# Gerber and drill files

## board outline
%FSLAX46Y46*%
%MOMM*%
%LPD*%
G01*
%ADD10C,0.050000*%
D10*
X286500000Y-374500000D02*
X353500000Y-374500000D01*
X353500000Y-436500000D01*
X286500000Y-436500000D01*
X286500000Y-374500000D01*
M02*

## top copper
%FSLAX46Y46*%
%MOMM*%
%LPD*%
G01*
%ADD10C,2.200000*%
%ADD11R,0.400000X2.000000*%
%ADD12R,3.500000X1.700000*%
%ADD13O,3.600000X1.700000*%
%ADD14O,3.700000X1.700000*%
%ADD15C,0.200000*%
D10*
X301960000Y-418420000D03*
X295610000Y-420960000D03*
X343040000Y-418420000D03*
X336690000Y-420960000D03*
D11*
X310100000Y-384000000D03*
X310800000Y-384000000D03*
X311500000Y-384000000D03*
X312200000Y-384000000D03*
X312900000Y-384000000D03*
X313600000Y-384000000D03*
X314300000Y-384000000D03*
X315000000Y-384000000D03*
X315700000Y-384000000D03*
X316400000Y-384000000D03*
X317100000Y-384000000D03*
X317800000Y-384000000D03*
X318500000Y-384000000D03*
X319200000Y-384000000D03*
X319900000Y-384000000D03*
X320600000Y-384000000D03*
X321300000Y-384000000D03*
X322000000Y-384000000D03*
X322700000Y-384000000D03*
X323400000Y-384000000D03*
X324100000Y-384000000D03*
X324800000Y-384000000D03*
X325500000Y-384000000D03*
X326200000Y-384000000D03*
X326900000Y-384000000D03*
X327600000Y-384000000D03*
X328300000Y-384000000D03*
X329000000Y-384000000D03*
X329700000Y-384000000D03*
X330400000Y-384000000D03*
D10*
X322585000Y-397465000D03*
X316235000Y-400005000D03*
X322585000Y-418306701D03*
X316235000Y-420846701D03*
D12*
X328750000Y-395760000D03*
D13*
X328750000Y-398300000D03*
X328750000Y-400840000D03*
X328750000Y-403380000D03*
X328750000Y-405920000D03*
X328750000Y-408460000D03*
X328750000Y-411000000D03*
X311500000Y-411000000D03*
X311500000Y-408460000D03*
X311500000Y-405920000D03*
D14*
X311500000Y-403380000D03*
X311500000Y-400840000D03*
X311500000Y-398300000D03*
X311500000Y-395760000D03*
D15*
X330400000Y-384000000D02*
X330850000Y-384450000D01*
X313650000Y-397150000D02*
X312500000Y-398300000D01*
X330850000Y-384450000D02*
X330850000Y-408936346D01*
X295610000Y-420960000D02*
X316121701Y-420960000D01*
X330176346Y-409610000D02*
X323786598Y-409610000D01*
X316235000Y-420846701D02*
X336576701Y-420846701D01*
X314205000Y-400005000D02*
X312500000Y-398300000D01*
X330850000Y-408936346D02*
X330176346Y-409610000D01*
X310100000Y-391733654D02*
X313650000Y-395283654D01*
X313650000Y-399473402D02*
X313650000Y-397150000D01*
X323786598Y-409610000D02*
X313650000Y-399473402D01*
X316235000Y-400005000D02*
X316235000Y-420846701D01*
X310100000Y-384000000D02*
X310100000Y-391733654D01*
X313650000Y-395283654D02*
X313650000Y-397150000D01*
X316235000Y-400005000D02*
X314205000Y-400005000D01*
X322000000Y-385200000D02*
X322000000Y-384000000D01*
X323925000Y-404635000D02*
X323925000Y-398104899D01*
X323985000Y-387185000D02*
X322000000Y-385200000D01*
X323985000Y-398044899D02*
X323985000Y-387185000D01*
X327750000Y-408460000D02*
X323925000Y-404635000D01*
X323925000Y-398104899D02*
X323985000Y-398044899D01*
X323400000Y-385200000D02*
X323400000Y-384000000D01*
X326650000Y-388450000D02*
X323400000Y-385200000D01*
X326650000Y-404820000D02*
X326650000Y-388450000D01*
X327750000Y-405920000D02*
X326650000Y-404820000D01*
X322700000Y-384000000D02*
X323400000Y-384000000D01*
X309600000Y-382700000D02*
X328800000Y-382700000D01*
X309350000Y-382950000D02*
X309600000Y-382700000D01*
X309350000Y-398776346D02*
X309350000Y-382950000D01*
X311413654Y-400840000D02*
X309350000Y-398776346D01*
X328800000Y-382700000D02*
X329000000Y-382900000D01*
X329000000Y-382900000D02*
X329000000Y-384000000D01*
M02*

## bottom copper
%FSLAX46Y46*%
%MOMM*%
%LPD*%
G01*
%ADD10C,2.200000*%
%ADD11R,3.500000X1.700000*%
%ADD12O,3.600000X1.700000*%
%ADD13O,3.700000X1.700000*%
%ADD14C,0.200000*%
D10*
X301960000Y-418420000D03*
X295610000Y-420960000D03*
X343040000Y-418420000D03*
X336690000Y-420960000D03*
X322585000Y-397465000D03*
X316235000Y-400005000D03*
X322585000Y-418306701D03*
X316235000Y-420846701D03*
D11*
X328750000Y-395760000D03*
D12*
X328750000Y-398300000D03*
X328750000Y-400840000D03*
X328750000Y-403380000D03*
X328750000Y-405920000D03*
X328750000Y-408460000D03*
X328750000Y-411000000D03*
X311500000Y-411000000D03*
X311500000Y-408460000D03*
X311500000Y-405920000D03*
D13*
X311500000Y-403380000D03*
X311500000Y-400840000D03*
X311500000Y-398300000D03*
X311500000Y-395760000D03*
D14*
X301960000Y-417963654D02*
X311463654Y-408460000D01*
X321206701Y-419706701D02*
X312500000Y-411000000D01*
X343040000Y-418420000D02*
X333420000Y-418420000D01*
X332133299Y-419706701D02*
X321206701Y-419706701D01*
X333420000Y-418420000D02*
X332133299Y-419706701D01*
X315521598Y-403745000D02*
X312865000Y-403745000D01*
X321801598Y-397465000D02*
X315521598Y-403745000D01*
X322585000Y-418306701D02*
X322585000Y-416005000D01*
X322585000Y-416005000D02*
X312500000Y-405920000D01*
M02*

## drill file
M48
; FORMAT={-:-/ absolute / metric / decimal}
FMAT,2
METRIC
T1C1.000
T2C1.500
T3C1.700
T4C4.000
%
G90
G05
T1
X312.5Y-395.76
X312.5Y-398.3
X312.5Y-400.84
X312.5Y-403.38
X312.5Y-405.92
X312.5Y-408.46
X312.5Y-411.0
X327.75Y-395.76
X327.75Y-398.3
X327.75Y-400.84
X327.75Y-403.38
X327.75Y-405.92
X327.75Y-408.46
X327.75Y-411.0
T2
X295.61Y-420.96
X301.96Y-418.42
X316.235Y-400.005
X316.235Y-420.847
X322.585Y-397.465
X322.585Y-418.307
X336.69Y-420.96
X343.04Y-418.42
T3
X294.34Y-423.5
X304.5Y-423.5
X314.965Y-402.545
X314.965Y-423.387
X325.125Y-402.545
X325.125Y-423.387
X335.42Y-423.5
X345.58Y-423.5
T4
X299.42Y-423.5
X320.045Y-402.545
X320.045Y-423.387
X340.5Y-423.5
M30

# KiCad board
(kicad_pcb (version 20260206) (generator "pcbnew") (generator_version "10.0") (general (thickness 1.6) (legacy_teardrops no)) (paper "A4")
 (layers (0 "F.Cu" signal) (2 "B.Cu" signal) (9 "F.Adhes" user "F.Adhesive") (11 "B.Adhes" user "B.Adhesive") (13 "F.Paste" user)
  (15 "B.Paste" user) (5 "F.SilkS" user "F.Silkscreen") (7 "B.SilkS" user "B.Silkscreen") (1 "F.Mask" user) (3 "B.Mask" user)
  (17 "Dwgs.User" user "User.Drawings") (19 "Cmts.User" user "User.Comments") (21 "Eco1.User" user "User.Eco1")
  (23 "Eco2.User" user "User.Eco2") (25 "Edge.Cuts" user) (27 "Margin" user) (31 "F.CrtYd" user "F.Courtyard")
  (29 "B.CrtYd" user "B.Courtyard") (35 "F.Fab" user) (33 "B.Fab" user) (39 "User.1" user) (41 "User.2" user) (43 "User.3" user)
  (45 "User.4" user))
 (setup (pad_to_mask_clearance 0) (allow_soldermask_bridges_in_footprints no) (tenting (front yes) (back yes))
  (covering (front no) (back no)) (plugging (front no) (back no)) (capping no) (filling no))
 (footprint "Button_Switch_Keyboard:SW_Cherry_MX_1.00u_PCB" (layer "F.Cu") (at 301.96 418.42)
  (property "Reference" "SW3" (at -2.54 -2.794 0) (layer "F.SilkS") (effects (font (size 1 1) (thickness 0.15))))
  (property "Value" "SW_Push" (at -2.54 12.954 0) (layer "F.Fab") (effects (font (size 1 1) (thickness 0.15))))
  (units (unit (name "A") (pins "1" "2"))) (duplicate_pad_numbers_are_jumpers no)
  (pad "" np_thru_hole circle (at -7.62 5.08) (size 1.7 1.7) (drill 1.7) (layers "*.Cu" "*.Mask"))
  (pad "" np_thru_hole circle (at -2.54 5.08) (size 4 4) (drill 4) (layers "*.Cu" "*.Mask"))
  (pad "" np_thru_hole circle (at 2.54 5.08) (size 1.7 1.7) (drill 1.7) (layers "*.Cu" "*.Mask"))
  (pad "1" thru_hole circle (at 0 0) (size 2.2 2.2) (drill 1.5) (layers "*.Cu" "*.Mask") (remove_unused_layers no)
   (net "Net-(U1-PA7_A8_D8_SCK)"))
  (pad "2" thru_hole circle (at -6.35 2.54) (size 2.2 2.2) (drill 1.5) (layers "*.Cu" "*.Mask") (remove_unused_layers no) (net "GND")))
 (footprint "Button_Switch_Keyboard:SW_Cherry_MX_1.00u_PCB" (layer "F.Cu") (at 343.04 418.42)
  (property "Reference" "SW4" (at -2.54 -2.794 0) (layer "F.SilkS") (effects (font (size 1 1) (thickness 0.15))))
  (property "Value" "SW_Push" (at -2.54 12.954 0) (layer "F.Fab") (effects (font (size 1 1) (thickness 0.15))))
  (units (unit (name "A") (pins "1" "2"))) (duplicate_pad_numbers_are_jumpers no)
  (pad "" np_thru_hole circle (at -7.62 5.08) (size 1.7 1.7) (drill 1.7) (layers "*.Cu" "*.Mask"))
  (pad "" np_thru_hole circle (at -2.54 5.08) (size 4 4) (drill 4) (layers "*.Cu" "*.Mask"))
  (pad "" np_thru_hole circle (at 2.54 5.08) (size 1.7 1.7) (drill 1.7) (layers "*.Cu" "*.Mask"))
  (pad "1" thru_hole circle (at 0 0) (size 2.2 2.2) (drill 1.5) (layers "*.Cu" "*.Mask") (remove_unused_layers no)
   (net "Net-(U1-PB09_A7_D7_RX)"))
  (pad "2" thru_hole circle (at -6.35 2.54) (size 2.2 2.2) (drill 1.5) (layers "*.Cu" "*.Mask") (remove_unused_layers no) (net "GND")))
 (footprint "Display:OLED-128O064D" (layer "F.Cu") (at 320.25 384)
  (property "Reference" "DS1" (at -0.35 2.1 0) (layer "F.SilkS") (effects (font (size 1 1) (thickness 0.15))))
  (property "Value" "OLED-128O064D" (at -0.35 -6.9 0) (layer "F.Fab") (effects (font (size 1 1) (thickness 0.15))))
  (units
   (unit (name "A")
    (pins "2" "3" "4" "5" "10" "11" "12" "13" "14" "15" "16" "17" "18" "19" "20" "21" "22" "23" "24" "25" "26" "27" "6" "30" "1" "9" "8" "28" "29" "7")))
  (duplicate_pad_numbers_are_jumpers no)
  (pad "1" smd rect (at -10.15 0) (size 0.4 2) (layers "F.Cu" "F.Mask" "F.Paste") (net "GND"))
  (pad "2" smd rect (at -9.45 0) (size 0.4 2) (layers "F.Cu" "F.Mask" "F.Paste") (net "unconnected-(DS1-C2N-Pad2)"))
  (pad "3" smd rect (at -8.75 0) (size 0.4 2) (layers "F.Cu" "F.Mask" "F.Paste") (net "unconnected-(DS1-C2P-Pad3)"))
  (pad "4" smd rect (at -8.05 0) (size 0.4 2) (layers "F.Cu" "F.Mask" "F.Paste") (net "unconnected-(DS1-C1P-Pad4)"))
  (pad "5" smd rect (at -7.35 0) (size 0.4 2) (layers "F.Cu" "F.Mask" "F.Paste") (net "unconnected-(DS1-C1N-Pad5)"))
  (pad "6" smd rect (at -6.65 0) (size 0.4 2) (layers "F.Cu" "F.Mask" "F.Paste") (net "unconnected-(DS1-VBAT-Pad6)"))
  (pad "7" smd rect (at -5.95 0) (size 0.4 2) (layers "F.Cu" "F.Mask" "F.Paste") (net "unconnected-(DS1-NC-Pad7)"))
  (pad "8" smd rect (at -5.25 0) (size 0.4 2) (layers "F.Cu" "F.Mask" "F.Paste") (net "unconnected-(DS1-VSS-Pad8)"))
  (pad "9" smd rect (at -4.55 0) (size 0.4 2) (layers "F.Cu" "F.Mask" "F.Paste") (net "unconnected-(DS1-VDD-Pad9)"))
  (pad "10" smd rect (at -3.85 0) (size 0.4 2) (layers "F.Cu" "F.Mask" "F.Paste") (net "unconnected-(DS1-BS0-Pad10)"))
  (pad "11" smd rect (at -3.15 0) (size 0.4 2) (layers "F.Cu" "F.Mask" "F.Paste") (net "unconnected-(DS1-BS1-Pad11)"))
  (pad "12" smd rect (at -2.45 0) (size 0.4 2) (layers "F.Cu" "F.Mask" "F.Paste") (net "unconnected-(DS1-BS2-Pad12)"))
  (pad "13" smd rect (at -1.75 0) (size 0.4 2) (layers "F.Cu" "F.Mask" "F.Paste") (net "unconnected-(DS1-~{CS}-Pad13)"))
  (pad "14" smd rect (at -1.05 0) (size 0.4 2) (layers "F.Cu" "F.Mask" "F.Paste") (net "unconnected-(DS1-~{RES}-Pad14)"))
  (pad "15" smd rect (at -0.35 0) (size 0.4 2) (layers "F.Cu" "F.Mask" "F.Paste") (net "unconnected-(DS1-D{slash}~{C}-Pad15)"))
  (pad "16" smd rect (at 0.35 0) (size 0.4 2) (layers "F.Cu" "F.Mask" "F.Paste") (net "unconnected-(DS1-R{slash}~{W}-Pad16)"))
  (pad "17" smd rect (at 1.05 0) (size 0.4 2) (layers "F.Cu" "F.Mask" "F.Paste") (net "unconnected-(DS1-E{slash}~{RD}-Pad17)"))
  (pad "18" smd rect (at 1.75 0) (size 0.4 2) (layers "F.Cu" "F.Mask" "F.Paste") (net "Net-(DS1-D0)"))
  (pad "19" smd rect (at 2.45 0) (size 0.4 2) (layers "F.Cu" "F.Mask" "F.Paste") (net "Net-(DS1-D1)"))
  (pad "20" smd rect (at 3.15 0) (size 0.4 2) (layers "F.Cu" "F.Mask" "F.Paste") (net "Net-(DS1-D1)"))
  (pad "21" smd rect (at 3.85 0) (size 0.4 2) (layers "F.Cu" "F.Mask" "F.Paste") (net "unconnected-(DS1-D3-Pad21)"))
  (pad "22" smd rect (at 4.55 0) (size 0.4 2) (layers "F.Cu" "F.Mask" "F.Paste") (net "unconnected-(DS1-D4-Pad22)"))
  (pad "23" smd rect (at 5.25 0) (size 0.4 2) (layers "F.Cu" "F.Mask" "F.Paste") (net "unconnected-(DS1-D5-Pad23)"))
  (pad "24" smd rect (at 5.95 0) (size 0.4 2) (layers "F.Cu" "F.Mask" "F.Paste") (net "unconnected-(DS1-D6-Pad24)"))
  (pad "25" smd rect (at 6.65 0) (size 0.4 2) (layers "F.Cu" "F.Mask" "F.Paste") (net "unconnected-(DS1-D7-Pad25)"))
  (pad "26" smd rect (at 7.35 0) (size 0.4 2) (layers "F.Cu" "F.Mask" "F.Paste") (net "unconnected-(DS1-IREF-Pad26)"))
  (pad "27" smd rect (at 8.05 0) (size 0.4 2) (layers "F.Cu" "F.Mask" "F.Paste") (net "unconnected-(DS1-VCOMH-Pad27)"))
  (pad "28" smd rect (at 8.75 0) (size 0.4 2) (layers "F.Cu" "F.Mask" "F.Paste") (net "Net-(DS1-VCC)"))
  (pad "29" smd rect (at 9.45 0) (size 0.4 2) (layers "F.Cu" "F.Mask" "F.Paste") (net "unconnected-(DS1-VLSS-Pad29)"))
  (pad "30" smd rect (at 10.15 0) (size 0.4 2) (layers "F.Cu" "F.Mask" "F.Paste") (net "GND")))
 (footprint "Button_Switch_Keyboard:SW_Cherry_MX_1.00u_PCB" (layer "F.Cu") (at 322.585 397.465)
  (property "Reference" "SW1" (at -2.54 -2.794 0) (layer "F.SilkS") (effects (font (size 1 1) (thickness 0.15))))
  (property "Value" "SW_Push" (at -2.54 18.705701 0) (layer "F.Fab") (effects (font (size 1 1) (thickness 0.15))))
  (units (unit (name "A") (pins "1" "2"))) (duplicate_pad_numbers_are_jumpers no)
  (pad "" np_thru_hole circle (at -7.62 5.08) (size 1.7 1.7) (drill 1.7) (layers "*.Cu" "*.Mask"))
  (pad "" np_thru_hole circle (at -2.54 5.08) (size 4 4) (drill 4) (layers "*.Cu" "*.Mask"))
  (pad "" np_thru_hole circle (at 2.54 5.08) (size 1.7 1.7) (drill 1.7) (layers "*.Cu" "*.Mask"))
  (pad "1" thru_hole circle (at 0 0) (size 2.2 2.2) (drill 1.5) (layers "*.Cu" "*.Mask") (remove_unused_layers no)
   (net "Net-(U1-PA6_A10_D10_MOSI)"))
  (pad "2" thru_hole circle (at -6.35 2.54) (size 2.2 2.2) (drill 1.5) (layers "*.Cu" "*.Mask") (remove_unused_layers no) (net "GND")))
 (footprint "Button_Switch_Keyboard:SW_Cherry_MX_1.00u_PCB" (layer "F.Cu") (at 322.585 418.306701)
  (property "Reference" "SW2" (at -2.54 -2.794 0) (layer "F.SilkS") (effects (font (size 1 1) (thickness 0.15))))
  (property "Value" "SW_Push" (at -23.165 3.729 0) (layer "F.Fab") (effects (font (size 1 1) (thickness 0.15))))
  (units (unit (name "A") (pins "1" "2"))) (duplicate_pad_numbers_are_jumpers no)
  (pad "" np_thru_hole circle (at -7.62 5.08) (size 1.7 1.7) (drill 1.7) (layers "*.Cu" "*.Mask"))
  (pad "" np_thru_hole circle (at -2.54 5.08) (size 4 4) (drill 4) (layers "*.Cu" "*.Mask"))
  (pad "" np_thru_hole circle (at 2.54 5.08) (size 1.7 1.7) (drill 1.7) (layers "*.Cu" "*.Mask"))
  (pad "1" thru_hole circle (at 0 0) (size 2.2 2.2) (drill 1.5) (layers "*.Cu" "*.Mask") (remove_unused_layers no)
   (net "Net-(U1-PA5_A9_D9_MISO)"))
  (pad "2" thru_hole circle (at -6.35 2.54) (size 2.2 2.2) (drill 1.5) (layers "*.Cu" "*.Mask") (remove_unused_layers no) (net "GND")))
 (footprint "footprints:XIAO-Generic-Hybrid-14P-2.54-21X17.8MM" (layer "B.Cu") (at 320.125 403.38 180)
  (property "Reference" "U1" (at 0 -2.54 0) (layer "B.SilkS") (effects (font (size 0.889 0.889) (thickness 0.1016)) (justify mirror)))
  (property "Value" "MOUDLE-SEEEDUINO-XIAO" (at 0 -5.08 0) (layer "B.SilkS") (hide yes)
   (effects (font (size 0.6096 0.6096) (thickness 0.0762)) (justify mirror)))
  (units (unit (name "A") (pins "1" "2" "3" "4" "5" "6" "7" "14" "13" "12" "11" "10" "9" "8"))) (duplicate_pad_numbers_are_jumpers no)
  (pad "1" thru_hole rect (at -7.625 7.62 180) (size 3.5 1.7) (drill 1 (offset -1 0)) (layers "*.Cu" "*.Mask") (remove_unused_layers no)
   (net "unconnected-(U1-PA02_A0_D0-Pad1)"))
  (pad "2" thru_hole oval (at -7.625 5.08 180) (size 3.6 1.7) (drill 1 (offset -1 0)) (layers "*.Cu" "*.Mask") (remove_unused_layers no)
   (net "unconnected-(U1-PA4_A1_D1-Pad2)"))
  (pad "3" thru_hole oval (at -7.625 2.54 180) (size 3.6 1.7) (drill 1 (offset -1 0)) (layers "*.Cu" "*.Mask") (remove_unused_layers no)
   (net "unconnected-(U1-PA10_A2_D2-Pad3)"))
  (pad "4" thru_hole oval (at -7.625 0 180) (size 3.6 1.7) (drill 1 (offset -1 0)) (layers "*.Cu" "*.Mask") (remove_unused_layers no)
   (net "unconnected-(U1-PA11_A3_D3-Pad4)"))
  (pad "5" thru_hole oval (at -7.625 -2.54 180) (size 3.6 1.7) (drill 1 (offset -1 0)) (layers "*.Cu" "*.Mask") (remove_unused_layers no)
   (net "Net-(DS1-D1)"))
  (pad "6" thru_hole oval (at -7.625 -5.08) (size 3.6 1.7) (drill 1 (offset 1 0)) (layers "*.Cu" "*.Mask") (remove_unused_layers no)
   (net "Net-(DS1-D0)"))
  (pad "7" thru_hole oval (at -7.625 -7.62 180) (size 3.6 1.7) (drill 1 (offset -1 0)) (layers "*.Cu" "*.Mask") (remove_unused_layers no)
   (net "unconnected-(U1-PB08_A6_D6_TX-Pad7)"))
  (pad "8" thru_hole oval (at 7.625 -7.62 180) (size 3.6 1.7) (drill 1 (offset 1 0)) (layers "*.Cu" "*.Mask") (remove_unused_layers no)
   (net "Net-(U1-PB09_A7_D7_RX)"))
  (pad "9" thru_hole oval (at 7.625 -5.08 180) (size 3.6 1.7) (drill 1 (offset 1 0)) (layers "*.Cu" "*.Mask") (remove_unused_layers no)
   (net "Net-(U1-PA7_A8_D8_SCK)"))
  (pad "10" thru_hole oval (at 7.625 -2.54 180) (size 3.6 1.7) (drill 1 (offset 1 0)) (layers "*.Cu" "*.Mask") (remove_unused_layers no)
   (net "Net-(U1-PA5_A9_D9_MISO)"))
  (pad "11" thru_hole oval (at 7.625 0 180) (size 3.7 1.7) (drill 1 (offset 1 0)) (layers "*.Cu" "*.Mask") (remove_unused_layers no)
   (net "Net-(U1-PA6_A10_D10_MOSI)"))
  (pad "12" thru_hole oval (at 7.625 2.54 180) (size 3.7 1.7) (drill 1 (offset 1 0)) (layers "*.Cu" "*.Mask") (remove_unused_layers no)
   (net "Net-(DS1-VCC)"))
  (pad "13" thru_hole oval (at 7.625 5.08 180) (size 3.7 1.7) (drill 1 (offset 1 0)) (layers "*.Cu" "*.Mask") (remove_unused_layers no)
   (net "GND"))
  (pad "14" thru_hole oval (at 7.625 7.62 180) (size 3.7 1.7) (drill 1 (offset 1 0)) (layers "*.Cu" "*.Mask") (remove_unused_layers no)
   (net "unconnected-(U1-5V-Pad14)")))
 (gr_rect (start 286.5 374.5) (end 353.5 436.5) (stroke (width 0.05) (type default)) (fill no) (layer "Edge.Cuts"))
 (segment (start 301.96 417.963654) (end 311.463654 408.46) (width 0.2) (layer "B.Cu") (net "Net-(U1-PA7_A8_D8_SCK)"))
 (segment (start 330.4 384) (end 330.85 384.45) (width 0.2) (layer "F.Cu") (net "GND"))
 (segment (start 313.65 397.15) (end 312.5 398.3) (width 0.2) (layer "F.Cu") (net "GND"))
 (segment (start 330.85 384.45) (end 330.85 408.936346) (width 0.2) (layer "F.Cu") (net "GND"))
 (segment (start 295.61 420.96) (end 316.121701 420.96) (width 0.2) (layer "F.Cu") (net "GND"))
 (segment (start 330.176346 409.61) (end 323.786598 409.61) (width 0.2) (layer "F.Cu") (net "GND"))
 (segment (start 316.235 420.846701) (end 336.576701 420.846701) (width 0.2) (layer "F.Cu") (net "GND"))
 (segment (start 314.205 400.005) (end 312.5 398.3) (width 0.2) (layer "F.Cu") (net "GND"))
 (segment (start 330.85 408.936346) (end 330.176346 409.61) (width 0.2) (layer "F.Cu") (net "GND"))
 (segment (start 310.1 391.733654) (end 313.65 395.283654) (width 0.2) (layer "F.Cu") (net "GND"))
 (segment (start 313.65 399.473402) (end 313.65 397.15) (width 0.2) (layer "F.Cu") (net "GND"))
 (segment (start 323.786598 409.61) (end 313.65 399.473402) (width 0.2) (layer "F.Cu") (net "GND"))
 (segment (start 316.235 400.005) (end 316.235 420.846701) (width 0.2) (layer "F.Cu") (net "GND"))
 (segment (start 310.1 384) (end 310.1 391.733654) (width 0.2) (layer "F.Cu") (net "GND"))
 (segment (start 313.65 395.283654) (end 313.65 397.15) (width 0.2) (layer "F.Cu") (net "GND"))
 (segment (start 316.235 400.005) (end 314.205 400.005) (width 0.2) (layer "F.Cu") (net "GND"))
 (segment (start 321.206701 419.706701) (end 312.5 411) (width 0.2) (layer "B.Cu") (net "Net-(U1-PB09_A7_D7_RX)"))
 (segment (start 343.04 418.42) (end 333.42 418.42) (width 0.2) (layer "B.Cu") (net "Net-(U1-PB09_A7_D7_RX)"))
 (segment (start 332.133299 419.706701) (end 321.206701 419.706701) (width 0.2) (layer "B.Cu") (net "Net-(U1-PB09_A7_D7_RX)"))
 (segment (start 333.42 418.42) (end 332.133299 419.706701) (width 0.2) (layer "B.Cu") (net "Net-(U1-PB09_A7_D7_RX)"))
 (segment (start 322 385.2) (end 322 384) (width 0.2) (layer "F.Cu") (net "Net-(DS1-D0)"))
 (segment (start 323.925 404.635) (end 323.925 398.104899) (width 0.2) (layer "F.Cu") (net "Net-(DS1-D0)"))
 (segment (start 323.985 387.185) (end 322 385.2) (width 0.2) (layer "F.Cu") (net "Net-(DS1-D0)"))
 (segment (start 323.985 398.044899) (end 323.985 387.185) (width 0.2) (layer "F.Cu") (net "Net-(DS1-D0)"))
 (segment (start 327.75 408.46) (end 323.925 404.635) (width 0.2) (layer "F.Cu") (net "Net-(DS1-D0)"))
 (segment (start 323.925 398.104899) (end 323.985 398.044899) (width 0.2) (layer "F.Cu") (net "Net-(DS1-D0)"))
 (segment (start 323.4 385.2) (end 323.4 384) (width 0.2) (layer "F.Cu") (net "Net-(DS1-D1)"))
 (segment (start 326.65 388.45) (end 323.4 385.2) (width 0.2) (layer "F.Cu") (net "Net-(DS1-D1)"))
 (segment (start 326.65 404.82) (end 326.65 388.45) (width 0.2) (layer "F.Cu") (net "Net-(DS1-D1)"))
 (segment (start 327.75 405.92) (end 326.65 404.82) (width 0.2) (layer "F.Cu") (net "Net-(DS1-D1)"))
 (segment (start 322.7 384) (end 323.4 384) (width 0.2) (layer "F.Cu") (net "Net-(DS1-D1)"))
 (segment (start 309.6 382.7) (end 328.8 382.7) (width 0.2) (layer "F.Cu") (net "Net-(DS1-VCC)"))
 (segment (start 309.35 382.95) (end 309.6 382.7) (width 0.2) (layer "F.Cu") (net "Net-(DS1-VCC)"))
 (segment (start 309.35 398.776346) (end 309.35 382.95) (width 0.2) (layer "F.Cu") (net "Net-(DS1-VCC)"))
 (segment (start 311.413654 400.84) (end 309.35 398.776346) (width 0.2) (layer "F.Cu") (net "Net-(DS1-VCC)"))
 (segment (start 328.8 382.7) (end 329 382.9) (width 0.2) (layer "F.Cu") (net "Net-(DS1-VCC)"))
 (segment (start 329 382.9) (end 329 384) (width 0.2) (layer "F.Cu") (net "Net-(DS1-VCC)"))
 (segment (start 315.521598 403.745) (end 312.865 403.745) (width 0.2) (layer "B.Cu") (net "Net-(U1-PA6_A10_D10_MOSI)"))
 (segment (start 321.801598 397.465) (end 315.521598 403.745) (width 0.2) (layer "B.Cu") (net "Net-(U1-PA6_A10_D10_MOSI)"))
 (segment (start 322.585 418.306701) (end 322.585 416.005) (width 0.2) (layer "B.Cu") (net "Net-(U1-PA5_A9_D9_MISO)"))
 (segment (start 322.585 416.005) (end 312.5 405.92) (width 0.2) (layer "B.Cu") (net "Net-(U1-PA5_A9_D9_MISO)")))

